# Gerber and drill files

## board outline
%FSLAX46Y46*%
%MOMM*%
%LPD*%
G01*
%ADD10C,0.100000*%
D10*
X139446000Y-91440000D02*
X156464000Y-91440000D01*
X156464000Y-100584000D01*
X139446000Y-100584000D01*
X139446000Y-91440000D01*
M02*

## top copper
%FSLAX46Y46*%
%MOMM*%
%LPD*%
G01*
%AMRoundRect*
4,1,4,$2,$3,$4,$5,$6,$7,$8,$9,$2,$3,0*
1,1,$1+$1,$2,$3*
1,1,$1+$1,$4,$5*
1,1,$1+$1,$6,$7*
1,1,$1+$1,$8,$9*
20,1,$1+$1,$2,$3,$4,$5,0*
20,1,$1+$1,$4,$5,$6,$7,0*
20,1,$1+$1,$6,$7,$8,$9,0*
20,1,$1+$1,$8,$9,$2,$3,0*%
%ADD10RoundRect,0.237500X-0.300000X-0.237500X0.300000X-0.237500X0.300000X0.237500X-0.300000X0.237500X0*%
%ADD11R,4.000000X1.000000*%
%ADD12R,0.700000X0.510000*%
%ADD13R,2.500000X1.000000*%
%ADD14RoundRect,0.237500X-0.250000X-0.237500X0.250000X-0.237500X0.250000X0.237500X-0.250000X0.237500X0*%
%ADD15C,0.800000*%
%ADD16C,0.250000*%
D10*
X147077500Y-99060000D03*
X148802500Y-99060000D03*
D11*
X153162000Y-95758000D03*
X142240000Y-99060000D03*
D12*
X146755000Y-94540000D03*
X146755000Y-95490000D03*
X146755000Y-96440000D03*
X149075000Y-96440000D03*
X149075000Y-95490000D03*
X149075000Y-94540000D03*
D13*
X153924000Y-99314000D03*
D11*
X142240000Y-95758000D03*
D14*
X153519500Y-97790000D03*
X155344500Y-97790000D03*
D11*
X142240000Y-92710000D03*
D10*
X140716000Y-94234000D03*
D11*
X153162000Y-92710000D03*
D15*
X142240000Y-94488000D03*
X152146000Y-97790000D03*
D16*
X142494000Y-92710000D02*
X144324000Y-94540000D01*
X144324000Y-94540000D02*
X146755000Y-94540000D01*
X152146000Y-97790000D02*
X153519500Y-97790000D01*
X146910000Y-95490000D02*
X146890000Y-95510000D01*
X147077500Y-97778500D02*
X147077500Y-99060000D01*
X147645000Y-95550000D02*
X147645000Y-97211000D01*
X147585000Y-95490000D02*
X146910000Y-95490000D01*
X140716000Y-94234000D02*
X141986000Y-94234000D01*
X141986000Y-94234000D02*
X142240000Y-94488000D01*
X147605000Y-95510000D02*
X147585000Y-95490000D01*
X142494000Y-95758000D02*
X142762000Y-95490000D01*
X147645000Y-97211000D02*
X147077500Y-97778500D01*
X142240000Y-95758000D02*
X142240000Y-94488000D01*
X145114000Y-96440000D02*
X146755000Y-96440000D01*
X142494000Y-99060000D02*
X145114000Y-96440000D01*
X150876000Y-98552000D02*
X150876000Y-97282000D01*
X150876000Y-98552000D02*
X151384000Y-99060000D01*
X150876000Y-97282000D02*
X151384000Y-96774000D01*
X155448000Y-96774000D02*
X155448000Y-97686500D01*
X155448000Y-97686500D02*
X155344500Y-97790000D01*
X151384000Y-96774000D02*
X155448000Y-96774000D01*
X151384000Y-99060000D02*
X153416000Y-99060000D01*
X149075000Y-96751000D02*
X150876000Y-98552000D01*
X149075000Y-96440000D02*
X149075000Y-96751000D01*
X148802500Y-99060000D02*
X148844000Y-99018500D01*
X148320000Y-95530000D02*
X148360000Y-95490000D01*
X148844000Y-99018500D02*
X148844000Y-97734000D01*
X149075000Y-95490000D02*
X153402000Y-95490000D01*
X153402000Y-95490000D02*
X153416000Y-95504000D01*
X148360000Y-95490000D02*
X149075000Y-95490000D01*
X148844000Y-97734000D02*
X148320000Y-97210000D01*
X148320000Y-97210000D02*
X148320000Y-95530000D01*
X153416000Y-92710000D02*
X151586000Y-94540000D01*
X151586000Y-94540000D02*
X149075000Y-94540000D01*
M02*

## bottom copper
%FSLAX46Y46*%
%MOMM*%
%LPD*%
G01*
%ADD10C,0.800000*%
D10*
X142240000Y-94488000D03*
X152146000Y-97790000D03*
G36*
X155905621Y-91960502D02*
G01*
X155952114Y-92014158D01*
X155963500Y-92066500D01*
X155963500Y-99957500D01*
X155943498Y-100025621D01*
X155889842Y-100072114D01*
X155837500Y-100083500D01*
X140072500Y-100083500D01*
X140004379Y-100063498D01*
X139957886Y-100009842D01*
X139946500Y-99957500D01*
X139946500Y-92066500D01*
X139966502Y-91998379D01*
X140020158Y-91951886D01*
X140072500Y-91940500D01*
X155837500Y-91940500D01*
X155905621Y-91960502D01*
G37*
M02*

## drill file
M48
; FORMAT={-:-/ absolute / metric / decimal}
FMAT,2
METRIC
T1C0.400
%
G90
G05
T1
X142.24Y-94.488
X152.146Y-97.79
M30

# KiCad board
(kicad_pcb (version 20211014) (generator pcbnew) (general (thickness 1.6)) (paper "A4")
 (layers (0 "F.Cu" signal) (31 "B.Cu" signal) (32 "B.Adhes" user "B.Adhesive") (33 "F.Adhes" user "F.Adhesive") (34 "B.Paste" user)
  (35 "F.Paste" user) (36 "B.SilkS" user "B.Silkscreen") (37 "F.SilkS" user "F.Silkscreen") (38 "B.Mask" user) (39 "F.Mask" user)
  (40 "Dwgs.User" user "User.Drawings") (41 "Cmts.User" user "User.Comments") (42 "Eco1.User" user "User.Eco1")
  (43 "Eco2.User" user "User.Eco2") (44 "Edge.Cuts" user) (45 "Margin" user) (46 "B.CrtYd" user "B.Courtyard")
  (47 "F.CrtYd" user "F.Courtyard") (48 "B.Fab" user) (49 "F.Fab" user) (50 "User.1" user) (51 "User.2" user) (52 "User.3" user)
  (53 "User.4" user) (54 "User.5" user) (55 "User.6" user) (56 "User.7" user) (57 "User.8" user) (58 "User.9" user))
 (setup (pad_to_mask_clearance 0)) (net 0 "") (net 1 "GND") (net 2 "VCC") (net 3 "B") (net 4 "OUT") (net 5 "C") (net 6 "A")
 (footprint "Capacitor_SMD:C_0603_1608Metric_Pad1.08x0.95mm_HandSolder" (layer "F.Cu") (at 147.94 99.06)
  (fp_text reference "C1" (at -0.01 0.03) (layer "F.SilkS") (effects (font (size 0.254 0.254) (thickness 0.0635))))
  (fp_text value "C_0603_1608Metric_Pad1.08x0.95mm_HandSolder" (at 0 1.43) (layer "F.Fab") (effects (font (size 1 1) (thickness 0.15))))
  (pad "1" smd roundrect (at -0.8625 0) (size 1.075 0.95) (layers "F.Cu" "F.Paste" "F.Mask") (roundrect_rratio 0.25) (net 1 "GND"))
  (pad "2" smd roundrect (at 0.8625 0) (size 1.075 0.95) (layers "F.Cu" "F.Paste" "F.Mask") (roundrect_rratio 0.25) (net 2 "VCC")))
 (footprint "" (layer "F.Cu") (at 153.162 95.758)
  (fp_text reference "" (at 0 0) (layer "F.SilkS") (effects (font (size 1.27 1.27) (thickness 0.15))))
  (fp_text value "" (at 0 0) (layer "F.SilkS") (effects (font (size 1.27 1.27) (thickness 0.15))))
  (pad "5" smd rect locked (at 0 0) (size 4 1) (layers "F.Cu" "F.Paste" "F.Mask") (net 2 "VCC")))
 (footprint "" (layer "F.Cu") (at 142.24 99.06)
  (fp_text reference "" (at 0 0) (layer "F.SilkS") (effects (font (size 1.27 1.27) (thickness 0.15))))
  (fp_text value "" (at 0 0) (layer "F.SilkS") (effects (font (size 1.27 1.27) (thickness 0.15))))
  (pad "3" smd rect locked (at 0 0) (size 4 1) (layers "F.Cu" "F.Paste" "F.Mask") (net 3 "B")))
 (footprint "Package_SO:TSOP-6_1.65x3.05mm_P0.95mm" (layer "F.Cu") (at 147.915 95.49)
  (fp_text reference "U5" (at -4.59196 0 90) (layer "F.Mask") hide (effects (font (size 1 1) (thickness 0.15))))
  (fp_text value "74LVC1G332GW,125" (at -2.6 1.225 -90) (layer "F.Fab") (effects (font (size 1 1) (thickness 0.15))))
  (pad "1" smd rect (at -1.16 -0.95) (size 0.7 0.51) (layers "F.Cu" "F.Paste" "F.Mask"))
  (pad "2" smd rect (at -1.16 0) (size 0.7 0.51) (layers "F.Cu" "F.Paste" "F.Mask") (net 1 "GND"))
  (pad "3" smd rect (at -1.16 0.95) (size 0.7 0.51) (layers "F.Cu" "F.Paste" "F.Mask") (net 3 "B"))
  (pad "4" smd rect (at 1.16 0.95) (size 0.7 0.51) (layers "F.Cu" "F.Paste" "F.Mask") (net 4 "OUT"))
  (pad "5" smd rect (at 1.16 0) (size 0.7 0.51) (layers "F.Cu" "F.Paste" "F.Mask") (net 2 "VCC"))
  (pad "6" smd rect (at 1.16 -0.95) (size 0.7 0.51) (layers "F.Cu" "F.Paste" "F.Mask") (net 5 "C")))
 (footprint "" (layer "F.Cu") (at 153.924 99.314)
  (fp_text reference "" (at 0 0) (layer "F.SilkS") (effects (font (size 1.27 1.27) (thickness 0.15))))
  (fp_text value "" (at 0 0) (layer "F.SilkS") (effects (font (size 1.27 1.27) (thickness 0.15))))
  (pad "4" smd rect locked (at 0 0) (size 2.5 1) (layers "F.Cu" "F.Paste" "F.Mask") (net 4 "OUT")))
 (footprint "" (layer "F.Cu") (at 142.24 95.758)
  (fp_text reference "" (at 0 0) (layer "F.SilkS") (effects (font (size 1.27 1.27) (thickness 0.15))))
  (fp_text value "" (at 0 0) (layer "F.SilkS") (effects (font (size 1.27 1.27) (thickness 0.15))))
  (pad "2" smd rect locked (at 0 0) (size 4 1) (layers "F.Cu" "F.Paste" "F.Mask") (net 1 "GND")))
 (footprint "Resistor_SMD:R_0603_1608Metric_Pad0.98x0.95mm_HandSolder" (layer "F.Cu") (at 154.432 97.79)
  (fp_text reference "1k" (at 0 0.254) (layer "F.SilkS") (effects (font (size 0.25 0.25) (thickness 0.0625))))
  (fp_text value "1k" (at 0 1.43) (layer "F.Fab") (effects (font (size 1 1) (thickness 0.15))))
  (pad "7" smd roundrect (at -0.9125 0) (size 0.975 0.95) (layers "F.Cu" "F.Paste" "F.Mask") (roundrect_rratio 0.25) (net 1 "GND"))
  (pad "8" smd roundrect (at 0.9125 0) (size 0.975 0.95) (layers "F.Cu" "F.Paste" "F.Mask") (roundrect_rratio 0.25) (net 4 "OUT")))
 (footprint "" (layer "F.Cu") (at 142.24 92.71)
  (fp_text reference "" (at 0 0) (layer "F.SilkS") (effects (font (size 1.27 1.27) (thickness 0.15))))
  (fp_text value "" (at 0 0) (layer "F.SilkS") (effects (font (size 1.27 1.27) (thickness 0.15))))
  (pad "1" smd rect locked (at 0 0) (size 4 1) (layers "F.Cu" "F.Paste" "F.Mask") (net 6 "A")))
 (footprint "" (layer "F.Cu") (at 140.716 94.234)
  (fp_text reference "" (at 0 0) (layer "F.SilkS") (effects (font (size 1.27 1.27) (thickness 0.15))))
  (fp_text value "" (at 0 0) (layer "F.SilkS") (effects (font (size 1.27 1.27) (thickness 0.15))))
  (pad "1" smd roundrect (at 0 0) (size 1.075 0.95) (layers "F.Cu" "F.Paste" "F.Mask") (roundrect_rratio 0.25) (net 1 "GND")))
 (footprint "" (layer "F.Cu") (at 153.162 92.71)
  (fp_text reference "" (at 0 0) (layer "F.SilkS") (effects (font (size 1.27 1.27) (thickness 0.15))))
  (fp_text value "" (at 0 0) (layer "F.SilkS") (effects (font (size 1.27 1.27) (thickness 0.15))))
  (pad "6" smd rect locked (at 0 0) (size 4 1) (layers "F.Cu" "F.Paste" "F.Mask") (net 5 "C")))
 (gr_rect (start 139.446 91.44) (end 156.464 100.584) (layer "Edge.Cuts") (width 0.1) (fill none))
 (segment (start 142.494 92.71) (end 144.324 94.54) (width 0.25) (layer "F.Cu") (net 6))
 (segment (start 144.324 94.54) (end 146.755 94.54) (width 0.25) (layer "F.Cu") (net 6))
 (segment (start 152.146 97.79) (end 153.5195 97.79) (width 0.25) (layer "F.Cu") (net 1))
 (segment (start 146.91 95.49) (end 146.89 95.51) (width 0.25) (layer "F.Cu") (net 1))
 (segment (start 147.0775 97.7785) (end 147.0775 99.06) (width 0.25) (layer "F.Cu") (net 1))
 (segment (start 147.645 95.55) (end 147.645 97.211) (width 0.25) (layer "F.Cu") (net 1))
 (segment (start 147.585 95.49) (end 146.91 95.49) (width 0.25) (layer "F.Cu") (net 1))
 (segment (start 140.716 94.234) (end 141.986 94.234) (width 0.25) (layer "F.Cu") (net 1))
 (segment (start 141.986 94.234) (end 142.24 94.488) (width 0.25) (layer "F.Cu") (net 1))
 (segment (start 147.605 95.51) (end 147.585 95.49) (width 0.25) (layer "F.Cu") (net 1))
 (segment (start 142.494 95.758) (end 142.762 95.49) (width 0.25) (layer "F.Cu") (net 1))
 (segment (start 147.645 97.211) (end 147.0775 97.7785) (width 0.25) (layer "F.Cu") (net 1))
 (segment (start 142.24 95.758) (end 142.24 94.488) (width 0.25) (layer "F.Cu") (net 1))
 (via (at 142.24 94.488) (size 0.8) (drill 0.4) (layers "F.Cu" "B.Cu") (free) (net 1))
 (via (at 152.146 97.79) (size 0.8) (drill 0.4) (layers "F.Cu" "B.Cu") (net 1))
 (segment (start 145.114 96.44) (end 146.755 96.44) (width 0.25) (layer "F.Cu") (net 3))
 (segment (start 142.494 99.06) (end 145.114 96.44) (width 0.25) (layer "F.Cu") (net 3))
 (segment (start 150.876 98.552) (end 150.876 97.282) (width 0.25) (layer "F.Cu") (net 4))
 (segment (start 150.876 98.552) (end 151.384 99.06) (width 0.25) (layer "F.Cu") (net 4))
 (segment (start 150.876 97.282) (end 151.384 96.774) (width 0.25) (layer "F.Cu") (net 4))
 (segment (start 155.448 96.774) (end 155.448 97.6865) (width 0.25) (layer "F.Cu") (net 4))
 (segment (start 155.448 97.6865) (end 155.3445 97.79) (width 0.25) (layer "F.Cu") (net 4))
 (segment (start 151.384 96.774) (end 155.448 96.774) (width 0.25) (layer "F.Cu") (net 4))
 (segment (start 151.384 99.06) (end 153.416 99.06) (width 0.25) (layer "F.Cu") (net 4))
 (segment (start 149.075 96.751) (end 150.876 98.552) (width 0.25) (layer "F.Cu") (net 4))
 (segment (start 149.075 96.44) (end 149.075 96.751) (width 0.25) (layer "F.Cu") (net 4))
 (segment (start 148.8025 99.06) (end 148.844 99.0185) (width 0.25) (layer "F.Cu") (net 2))
 (segment (start 148.32 95.53) (end 148.36 95.49) (width 0.25) (layer "F.Cu") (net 2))
 (segment (start 148.844 99.0185) (end 148.844 97.734) (width 0.25) (layer "F.Cu") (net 2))
 (segment (start 149.075 95.49) (end 153.402 95.49) (width 0.25) (layer "F.Cu") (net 2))
 (segment (start 153.402 95.49) (end 153.416 95.504) (width 0.25) (layer "F.Cu") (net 2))
 (segment (start 148.36 95.49) (end 149.075 95.49) (width 0.25) (layer "F.Cu") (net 2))
 (segment (start 148.844 97.734) (end 148.32 97.21) (width 0.25) (layer "F.Cu") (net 2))
 (segment (start 148.32 97.21) (end 148.32 95.53) (width 0.25) (layer "F.Cu") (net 2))
 (segment (start 153.416 92.71) (end 151.586 94.54) (width 0.25) (layer "F.Cu") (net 5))
 (segment (start 151.586 94.54) (end 149.075 94.54) (width 0.25) (layer "F.Cu") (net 5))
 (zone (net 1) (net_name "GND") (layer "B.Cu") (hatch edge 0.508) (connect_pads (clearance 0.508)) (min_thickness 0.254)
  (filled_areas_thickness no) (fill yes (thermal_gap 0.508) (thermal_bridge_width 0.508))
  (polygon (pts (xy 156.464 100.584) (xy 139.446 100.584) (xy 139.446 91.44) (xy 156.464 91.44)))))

